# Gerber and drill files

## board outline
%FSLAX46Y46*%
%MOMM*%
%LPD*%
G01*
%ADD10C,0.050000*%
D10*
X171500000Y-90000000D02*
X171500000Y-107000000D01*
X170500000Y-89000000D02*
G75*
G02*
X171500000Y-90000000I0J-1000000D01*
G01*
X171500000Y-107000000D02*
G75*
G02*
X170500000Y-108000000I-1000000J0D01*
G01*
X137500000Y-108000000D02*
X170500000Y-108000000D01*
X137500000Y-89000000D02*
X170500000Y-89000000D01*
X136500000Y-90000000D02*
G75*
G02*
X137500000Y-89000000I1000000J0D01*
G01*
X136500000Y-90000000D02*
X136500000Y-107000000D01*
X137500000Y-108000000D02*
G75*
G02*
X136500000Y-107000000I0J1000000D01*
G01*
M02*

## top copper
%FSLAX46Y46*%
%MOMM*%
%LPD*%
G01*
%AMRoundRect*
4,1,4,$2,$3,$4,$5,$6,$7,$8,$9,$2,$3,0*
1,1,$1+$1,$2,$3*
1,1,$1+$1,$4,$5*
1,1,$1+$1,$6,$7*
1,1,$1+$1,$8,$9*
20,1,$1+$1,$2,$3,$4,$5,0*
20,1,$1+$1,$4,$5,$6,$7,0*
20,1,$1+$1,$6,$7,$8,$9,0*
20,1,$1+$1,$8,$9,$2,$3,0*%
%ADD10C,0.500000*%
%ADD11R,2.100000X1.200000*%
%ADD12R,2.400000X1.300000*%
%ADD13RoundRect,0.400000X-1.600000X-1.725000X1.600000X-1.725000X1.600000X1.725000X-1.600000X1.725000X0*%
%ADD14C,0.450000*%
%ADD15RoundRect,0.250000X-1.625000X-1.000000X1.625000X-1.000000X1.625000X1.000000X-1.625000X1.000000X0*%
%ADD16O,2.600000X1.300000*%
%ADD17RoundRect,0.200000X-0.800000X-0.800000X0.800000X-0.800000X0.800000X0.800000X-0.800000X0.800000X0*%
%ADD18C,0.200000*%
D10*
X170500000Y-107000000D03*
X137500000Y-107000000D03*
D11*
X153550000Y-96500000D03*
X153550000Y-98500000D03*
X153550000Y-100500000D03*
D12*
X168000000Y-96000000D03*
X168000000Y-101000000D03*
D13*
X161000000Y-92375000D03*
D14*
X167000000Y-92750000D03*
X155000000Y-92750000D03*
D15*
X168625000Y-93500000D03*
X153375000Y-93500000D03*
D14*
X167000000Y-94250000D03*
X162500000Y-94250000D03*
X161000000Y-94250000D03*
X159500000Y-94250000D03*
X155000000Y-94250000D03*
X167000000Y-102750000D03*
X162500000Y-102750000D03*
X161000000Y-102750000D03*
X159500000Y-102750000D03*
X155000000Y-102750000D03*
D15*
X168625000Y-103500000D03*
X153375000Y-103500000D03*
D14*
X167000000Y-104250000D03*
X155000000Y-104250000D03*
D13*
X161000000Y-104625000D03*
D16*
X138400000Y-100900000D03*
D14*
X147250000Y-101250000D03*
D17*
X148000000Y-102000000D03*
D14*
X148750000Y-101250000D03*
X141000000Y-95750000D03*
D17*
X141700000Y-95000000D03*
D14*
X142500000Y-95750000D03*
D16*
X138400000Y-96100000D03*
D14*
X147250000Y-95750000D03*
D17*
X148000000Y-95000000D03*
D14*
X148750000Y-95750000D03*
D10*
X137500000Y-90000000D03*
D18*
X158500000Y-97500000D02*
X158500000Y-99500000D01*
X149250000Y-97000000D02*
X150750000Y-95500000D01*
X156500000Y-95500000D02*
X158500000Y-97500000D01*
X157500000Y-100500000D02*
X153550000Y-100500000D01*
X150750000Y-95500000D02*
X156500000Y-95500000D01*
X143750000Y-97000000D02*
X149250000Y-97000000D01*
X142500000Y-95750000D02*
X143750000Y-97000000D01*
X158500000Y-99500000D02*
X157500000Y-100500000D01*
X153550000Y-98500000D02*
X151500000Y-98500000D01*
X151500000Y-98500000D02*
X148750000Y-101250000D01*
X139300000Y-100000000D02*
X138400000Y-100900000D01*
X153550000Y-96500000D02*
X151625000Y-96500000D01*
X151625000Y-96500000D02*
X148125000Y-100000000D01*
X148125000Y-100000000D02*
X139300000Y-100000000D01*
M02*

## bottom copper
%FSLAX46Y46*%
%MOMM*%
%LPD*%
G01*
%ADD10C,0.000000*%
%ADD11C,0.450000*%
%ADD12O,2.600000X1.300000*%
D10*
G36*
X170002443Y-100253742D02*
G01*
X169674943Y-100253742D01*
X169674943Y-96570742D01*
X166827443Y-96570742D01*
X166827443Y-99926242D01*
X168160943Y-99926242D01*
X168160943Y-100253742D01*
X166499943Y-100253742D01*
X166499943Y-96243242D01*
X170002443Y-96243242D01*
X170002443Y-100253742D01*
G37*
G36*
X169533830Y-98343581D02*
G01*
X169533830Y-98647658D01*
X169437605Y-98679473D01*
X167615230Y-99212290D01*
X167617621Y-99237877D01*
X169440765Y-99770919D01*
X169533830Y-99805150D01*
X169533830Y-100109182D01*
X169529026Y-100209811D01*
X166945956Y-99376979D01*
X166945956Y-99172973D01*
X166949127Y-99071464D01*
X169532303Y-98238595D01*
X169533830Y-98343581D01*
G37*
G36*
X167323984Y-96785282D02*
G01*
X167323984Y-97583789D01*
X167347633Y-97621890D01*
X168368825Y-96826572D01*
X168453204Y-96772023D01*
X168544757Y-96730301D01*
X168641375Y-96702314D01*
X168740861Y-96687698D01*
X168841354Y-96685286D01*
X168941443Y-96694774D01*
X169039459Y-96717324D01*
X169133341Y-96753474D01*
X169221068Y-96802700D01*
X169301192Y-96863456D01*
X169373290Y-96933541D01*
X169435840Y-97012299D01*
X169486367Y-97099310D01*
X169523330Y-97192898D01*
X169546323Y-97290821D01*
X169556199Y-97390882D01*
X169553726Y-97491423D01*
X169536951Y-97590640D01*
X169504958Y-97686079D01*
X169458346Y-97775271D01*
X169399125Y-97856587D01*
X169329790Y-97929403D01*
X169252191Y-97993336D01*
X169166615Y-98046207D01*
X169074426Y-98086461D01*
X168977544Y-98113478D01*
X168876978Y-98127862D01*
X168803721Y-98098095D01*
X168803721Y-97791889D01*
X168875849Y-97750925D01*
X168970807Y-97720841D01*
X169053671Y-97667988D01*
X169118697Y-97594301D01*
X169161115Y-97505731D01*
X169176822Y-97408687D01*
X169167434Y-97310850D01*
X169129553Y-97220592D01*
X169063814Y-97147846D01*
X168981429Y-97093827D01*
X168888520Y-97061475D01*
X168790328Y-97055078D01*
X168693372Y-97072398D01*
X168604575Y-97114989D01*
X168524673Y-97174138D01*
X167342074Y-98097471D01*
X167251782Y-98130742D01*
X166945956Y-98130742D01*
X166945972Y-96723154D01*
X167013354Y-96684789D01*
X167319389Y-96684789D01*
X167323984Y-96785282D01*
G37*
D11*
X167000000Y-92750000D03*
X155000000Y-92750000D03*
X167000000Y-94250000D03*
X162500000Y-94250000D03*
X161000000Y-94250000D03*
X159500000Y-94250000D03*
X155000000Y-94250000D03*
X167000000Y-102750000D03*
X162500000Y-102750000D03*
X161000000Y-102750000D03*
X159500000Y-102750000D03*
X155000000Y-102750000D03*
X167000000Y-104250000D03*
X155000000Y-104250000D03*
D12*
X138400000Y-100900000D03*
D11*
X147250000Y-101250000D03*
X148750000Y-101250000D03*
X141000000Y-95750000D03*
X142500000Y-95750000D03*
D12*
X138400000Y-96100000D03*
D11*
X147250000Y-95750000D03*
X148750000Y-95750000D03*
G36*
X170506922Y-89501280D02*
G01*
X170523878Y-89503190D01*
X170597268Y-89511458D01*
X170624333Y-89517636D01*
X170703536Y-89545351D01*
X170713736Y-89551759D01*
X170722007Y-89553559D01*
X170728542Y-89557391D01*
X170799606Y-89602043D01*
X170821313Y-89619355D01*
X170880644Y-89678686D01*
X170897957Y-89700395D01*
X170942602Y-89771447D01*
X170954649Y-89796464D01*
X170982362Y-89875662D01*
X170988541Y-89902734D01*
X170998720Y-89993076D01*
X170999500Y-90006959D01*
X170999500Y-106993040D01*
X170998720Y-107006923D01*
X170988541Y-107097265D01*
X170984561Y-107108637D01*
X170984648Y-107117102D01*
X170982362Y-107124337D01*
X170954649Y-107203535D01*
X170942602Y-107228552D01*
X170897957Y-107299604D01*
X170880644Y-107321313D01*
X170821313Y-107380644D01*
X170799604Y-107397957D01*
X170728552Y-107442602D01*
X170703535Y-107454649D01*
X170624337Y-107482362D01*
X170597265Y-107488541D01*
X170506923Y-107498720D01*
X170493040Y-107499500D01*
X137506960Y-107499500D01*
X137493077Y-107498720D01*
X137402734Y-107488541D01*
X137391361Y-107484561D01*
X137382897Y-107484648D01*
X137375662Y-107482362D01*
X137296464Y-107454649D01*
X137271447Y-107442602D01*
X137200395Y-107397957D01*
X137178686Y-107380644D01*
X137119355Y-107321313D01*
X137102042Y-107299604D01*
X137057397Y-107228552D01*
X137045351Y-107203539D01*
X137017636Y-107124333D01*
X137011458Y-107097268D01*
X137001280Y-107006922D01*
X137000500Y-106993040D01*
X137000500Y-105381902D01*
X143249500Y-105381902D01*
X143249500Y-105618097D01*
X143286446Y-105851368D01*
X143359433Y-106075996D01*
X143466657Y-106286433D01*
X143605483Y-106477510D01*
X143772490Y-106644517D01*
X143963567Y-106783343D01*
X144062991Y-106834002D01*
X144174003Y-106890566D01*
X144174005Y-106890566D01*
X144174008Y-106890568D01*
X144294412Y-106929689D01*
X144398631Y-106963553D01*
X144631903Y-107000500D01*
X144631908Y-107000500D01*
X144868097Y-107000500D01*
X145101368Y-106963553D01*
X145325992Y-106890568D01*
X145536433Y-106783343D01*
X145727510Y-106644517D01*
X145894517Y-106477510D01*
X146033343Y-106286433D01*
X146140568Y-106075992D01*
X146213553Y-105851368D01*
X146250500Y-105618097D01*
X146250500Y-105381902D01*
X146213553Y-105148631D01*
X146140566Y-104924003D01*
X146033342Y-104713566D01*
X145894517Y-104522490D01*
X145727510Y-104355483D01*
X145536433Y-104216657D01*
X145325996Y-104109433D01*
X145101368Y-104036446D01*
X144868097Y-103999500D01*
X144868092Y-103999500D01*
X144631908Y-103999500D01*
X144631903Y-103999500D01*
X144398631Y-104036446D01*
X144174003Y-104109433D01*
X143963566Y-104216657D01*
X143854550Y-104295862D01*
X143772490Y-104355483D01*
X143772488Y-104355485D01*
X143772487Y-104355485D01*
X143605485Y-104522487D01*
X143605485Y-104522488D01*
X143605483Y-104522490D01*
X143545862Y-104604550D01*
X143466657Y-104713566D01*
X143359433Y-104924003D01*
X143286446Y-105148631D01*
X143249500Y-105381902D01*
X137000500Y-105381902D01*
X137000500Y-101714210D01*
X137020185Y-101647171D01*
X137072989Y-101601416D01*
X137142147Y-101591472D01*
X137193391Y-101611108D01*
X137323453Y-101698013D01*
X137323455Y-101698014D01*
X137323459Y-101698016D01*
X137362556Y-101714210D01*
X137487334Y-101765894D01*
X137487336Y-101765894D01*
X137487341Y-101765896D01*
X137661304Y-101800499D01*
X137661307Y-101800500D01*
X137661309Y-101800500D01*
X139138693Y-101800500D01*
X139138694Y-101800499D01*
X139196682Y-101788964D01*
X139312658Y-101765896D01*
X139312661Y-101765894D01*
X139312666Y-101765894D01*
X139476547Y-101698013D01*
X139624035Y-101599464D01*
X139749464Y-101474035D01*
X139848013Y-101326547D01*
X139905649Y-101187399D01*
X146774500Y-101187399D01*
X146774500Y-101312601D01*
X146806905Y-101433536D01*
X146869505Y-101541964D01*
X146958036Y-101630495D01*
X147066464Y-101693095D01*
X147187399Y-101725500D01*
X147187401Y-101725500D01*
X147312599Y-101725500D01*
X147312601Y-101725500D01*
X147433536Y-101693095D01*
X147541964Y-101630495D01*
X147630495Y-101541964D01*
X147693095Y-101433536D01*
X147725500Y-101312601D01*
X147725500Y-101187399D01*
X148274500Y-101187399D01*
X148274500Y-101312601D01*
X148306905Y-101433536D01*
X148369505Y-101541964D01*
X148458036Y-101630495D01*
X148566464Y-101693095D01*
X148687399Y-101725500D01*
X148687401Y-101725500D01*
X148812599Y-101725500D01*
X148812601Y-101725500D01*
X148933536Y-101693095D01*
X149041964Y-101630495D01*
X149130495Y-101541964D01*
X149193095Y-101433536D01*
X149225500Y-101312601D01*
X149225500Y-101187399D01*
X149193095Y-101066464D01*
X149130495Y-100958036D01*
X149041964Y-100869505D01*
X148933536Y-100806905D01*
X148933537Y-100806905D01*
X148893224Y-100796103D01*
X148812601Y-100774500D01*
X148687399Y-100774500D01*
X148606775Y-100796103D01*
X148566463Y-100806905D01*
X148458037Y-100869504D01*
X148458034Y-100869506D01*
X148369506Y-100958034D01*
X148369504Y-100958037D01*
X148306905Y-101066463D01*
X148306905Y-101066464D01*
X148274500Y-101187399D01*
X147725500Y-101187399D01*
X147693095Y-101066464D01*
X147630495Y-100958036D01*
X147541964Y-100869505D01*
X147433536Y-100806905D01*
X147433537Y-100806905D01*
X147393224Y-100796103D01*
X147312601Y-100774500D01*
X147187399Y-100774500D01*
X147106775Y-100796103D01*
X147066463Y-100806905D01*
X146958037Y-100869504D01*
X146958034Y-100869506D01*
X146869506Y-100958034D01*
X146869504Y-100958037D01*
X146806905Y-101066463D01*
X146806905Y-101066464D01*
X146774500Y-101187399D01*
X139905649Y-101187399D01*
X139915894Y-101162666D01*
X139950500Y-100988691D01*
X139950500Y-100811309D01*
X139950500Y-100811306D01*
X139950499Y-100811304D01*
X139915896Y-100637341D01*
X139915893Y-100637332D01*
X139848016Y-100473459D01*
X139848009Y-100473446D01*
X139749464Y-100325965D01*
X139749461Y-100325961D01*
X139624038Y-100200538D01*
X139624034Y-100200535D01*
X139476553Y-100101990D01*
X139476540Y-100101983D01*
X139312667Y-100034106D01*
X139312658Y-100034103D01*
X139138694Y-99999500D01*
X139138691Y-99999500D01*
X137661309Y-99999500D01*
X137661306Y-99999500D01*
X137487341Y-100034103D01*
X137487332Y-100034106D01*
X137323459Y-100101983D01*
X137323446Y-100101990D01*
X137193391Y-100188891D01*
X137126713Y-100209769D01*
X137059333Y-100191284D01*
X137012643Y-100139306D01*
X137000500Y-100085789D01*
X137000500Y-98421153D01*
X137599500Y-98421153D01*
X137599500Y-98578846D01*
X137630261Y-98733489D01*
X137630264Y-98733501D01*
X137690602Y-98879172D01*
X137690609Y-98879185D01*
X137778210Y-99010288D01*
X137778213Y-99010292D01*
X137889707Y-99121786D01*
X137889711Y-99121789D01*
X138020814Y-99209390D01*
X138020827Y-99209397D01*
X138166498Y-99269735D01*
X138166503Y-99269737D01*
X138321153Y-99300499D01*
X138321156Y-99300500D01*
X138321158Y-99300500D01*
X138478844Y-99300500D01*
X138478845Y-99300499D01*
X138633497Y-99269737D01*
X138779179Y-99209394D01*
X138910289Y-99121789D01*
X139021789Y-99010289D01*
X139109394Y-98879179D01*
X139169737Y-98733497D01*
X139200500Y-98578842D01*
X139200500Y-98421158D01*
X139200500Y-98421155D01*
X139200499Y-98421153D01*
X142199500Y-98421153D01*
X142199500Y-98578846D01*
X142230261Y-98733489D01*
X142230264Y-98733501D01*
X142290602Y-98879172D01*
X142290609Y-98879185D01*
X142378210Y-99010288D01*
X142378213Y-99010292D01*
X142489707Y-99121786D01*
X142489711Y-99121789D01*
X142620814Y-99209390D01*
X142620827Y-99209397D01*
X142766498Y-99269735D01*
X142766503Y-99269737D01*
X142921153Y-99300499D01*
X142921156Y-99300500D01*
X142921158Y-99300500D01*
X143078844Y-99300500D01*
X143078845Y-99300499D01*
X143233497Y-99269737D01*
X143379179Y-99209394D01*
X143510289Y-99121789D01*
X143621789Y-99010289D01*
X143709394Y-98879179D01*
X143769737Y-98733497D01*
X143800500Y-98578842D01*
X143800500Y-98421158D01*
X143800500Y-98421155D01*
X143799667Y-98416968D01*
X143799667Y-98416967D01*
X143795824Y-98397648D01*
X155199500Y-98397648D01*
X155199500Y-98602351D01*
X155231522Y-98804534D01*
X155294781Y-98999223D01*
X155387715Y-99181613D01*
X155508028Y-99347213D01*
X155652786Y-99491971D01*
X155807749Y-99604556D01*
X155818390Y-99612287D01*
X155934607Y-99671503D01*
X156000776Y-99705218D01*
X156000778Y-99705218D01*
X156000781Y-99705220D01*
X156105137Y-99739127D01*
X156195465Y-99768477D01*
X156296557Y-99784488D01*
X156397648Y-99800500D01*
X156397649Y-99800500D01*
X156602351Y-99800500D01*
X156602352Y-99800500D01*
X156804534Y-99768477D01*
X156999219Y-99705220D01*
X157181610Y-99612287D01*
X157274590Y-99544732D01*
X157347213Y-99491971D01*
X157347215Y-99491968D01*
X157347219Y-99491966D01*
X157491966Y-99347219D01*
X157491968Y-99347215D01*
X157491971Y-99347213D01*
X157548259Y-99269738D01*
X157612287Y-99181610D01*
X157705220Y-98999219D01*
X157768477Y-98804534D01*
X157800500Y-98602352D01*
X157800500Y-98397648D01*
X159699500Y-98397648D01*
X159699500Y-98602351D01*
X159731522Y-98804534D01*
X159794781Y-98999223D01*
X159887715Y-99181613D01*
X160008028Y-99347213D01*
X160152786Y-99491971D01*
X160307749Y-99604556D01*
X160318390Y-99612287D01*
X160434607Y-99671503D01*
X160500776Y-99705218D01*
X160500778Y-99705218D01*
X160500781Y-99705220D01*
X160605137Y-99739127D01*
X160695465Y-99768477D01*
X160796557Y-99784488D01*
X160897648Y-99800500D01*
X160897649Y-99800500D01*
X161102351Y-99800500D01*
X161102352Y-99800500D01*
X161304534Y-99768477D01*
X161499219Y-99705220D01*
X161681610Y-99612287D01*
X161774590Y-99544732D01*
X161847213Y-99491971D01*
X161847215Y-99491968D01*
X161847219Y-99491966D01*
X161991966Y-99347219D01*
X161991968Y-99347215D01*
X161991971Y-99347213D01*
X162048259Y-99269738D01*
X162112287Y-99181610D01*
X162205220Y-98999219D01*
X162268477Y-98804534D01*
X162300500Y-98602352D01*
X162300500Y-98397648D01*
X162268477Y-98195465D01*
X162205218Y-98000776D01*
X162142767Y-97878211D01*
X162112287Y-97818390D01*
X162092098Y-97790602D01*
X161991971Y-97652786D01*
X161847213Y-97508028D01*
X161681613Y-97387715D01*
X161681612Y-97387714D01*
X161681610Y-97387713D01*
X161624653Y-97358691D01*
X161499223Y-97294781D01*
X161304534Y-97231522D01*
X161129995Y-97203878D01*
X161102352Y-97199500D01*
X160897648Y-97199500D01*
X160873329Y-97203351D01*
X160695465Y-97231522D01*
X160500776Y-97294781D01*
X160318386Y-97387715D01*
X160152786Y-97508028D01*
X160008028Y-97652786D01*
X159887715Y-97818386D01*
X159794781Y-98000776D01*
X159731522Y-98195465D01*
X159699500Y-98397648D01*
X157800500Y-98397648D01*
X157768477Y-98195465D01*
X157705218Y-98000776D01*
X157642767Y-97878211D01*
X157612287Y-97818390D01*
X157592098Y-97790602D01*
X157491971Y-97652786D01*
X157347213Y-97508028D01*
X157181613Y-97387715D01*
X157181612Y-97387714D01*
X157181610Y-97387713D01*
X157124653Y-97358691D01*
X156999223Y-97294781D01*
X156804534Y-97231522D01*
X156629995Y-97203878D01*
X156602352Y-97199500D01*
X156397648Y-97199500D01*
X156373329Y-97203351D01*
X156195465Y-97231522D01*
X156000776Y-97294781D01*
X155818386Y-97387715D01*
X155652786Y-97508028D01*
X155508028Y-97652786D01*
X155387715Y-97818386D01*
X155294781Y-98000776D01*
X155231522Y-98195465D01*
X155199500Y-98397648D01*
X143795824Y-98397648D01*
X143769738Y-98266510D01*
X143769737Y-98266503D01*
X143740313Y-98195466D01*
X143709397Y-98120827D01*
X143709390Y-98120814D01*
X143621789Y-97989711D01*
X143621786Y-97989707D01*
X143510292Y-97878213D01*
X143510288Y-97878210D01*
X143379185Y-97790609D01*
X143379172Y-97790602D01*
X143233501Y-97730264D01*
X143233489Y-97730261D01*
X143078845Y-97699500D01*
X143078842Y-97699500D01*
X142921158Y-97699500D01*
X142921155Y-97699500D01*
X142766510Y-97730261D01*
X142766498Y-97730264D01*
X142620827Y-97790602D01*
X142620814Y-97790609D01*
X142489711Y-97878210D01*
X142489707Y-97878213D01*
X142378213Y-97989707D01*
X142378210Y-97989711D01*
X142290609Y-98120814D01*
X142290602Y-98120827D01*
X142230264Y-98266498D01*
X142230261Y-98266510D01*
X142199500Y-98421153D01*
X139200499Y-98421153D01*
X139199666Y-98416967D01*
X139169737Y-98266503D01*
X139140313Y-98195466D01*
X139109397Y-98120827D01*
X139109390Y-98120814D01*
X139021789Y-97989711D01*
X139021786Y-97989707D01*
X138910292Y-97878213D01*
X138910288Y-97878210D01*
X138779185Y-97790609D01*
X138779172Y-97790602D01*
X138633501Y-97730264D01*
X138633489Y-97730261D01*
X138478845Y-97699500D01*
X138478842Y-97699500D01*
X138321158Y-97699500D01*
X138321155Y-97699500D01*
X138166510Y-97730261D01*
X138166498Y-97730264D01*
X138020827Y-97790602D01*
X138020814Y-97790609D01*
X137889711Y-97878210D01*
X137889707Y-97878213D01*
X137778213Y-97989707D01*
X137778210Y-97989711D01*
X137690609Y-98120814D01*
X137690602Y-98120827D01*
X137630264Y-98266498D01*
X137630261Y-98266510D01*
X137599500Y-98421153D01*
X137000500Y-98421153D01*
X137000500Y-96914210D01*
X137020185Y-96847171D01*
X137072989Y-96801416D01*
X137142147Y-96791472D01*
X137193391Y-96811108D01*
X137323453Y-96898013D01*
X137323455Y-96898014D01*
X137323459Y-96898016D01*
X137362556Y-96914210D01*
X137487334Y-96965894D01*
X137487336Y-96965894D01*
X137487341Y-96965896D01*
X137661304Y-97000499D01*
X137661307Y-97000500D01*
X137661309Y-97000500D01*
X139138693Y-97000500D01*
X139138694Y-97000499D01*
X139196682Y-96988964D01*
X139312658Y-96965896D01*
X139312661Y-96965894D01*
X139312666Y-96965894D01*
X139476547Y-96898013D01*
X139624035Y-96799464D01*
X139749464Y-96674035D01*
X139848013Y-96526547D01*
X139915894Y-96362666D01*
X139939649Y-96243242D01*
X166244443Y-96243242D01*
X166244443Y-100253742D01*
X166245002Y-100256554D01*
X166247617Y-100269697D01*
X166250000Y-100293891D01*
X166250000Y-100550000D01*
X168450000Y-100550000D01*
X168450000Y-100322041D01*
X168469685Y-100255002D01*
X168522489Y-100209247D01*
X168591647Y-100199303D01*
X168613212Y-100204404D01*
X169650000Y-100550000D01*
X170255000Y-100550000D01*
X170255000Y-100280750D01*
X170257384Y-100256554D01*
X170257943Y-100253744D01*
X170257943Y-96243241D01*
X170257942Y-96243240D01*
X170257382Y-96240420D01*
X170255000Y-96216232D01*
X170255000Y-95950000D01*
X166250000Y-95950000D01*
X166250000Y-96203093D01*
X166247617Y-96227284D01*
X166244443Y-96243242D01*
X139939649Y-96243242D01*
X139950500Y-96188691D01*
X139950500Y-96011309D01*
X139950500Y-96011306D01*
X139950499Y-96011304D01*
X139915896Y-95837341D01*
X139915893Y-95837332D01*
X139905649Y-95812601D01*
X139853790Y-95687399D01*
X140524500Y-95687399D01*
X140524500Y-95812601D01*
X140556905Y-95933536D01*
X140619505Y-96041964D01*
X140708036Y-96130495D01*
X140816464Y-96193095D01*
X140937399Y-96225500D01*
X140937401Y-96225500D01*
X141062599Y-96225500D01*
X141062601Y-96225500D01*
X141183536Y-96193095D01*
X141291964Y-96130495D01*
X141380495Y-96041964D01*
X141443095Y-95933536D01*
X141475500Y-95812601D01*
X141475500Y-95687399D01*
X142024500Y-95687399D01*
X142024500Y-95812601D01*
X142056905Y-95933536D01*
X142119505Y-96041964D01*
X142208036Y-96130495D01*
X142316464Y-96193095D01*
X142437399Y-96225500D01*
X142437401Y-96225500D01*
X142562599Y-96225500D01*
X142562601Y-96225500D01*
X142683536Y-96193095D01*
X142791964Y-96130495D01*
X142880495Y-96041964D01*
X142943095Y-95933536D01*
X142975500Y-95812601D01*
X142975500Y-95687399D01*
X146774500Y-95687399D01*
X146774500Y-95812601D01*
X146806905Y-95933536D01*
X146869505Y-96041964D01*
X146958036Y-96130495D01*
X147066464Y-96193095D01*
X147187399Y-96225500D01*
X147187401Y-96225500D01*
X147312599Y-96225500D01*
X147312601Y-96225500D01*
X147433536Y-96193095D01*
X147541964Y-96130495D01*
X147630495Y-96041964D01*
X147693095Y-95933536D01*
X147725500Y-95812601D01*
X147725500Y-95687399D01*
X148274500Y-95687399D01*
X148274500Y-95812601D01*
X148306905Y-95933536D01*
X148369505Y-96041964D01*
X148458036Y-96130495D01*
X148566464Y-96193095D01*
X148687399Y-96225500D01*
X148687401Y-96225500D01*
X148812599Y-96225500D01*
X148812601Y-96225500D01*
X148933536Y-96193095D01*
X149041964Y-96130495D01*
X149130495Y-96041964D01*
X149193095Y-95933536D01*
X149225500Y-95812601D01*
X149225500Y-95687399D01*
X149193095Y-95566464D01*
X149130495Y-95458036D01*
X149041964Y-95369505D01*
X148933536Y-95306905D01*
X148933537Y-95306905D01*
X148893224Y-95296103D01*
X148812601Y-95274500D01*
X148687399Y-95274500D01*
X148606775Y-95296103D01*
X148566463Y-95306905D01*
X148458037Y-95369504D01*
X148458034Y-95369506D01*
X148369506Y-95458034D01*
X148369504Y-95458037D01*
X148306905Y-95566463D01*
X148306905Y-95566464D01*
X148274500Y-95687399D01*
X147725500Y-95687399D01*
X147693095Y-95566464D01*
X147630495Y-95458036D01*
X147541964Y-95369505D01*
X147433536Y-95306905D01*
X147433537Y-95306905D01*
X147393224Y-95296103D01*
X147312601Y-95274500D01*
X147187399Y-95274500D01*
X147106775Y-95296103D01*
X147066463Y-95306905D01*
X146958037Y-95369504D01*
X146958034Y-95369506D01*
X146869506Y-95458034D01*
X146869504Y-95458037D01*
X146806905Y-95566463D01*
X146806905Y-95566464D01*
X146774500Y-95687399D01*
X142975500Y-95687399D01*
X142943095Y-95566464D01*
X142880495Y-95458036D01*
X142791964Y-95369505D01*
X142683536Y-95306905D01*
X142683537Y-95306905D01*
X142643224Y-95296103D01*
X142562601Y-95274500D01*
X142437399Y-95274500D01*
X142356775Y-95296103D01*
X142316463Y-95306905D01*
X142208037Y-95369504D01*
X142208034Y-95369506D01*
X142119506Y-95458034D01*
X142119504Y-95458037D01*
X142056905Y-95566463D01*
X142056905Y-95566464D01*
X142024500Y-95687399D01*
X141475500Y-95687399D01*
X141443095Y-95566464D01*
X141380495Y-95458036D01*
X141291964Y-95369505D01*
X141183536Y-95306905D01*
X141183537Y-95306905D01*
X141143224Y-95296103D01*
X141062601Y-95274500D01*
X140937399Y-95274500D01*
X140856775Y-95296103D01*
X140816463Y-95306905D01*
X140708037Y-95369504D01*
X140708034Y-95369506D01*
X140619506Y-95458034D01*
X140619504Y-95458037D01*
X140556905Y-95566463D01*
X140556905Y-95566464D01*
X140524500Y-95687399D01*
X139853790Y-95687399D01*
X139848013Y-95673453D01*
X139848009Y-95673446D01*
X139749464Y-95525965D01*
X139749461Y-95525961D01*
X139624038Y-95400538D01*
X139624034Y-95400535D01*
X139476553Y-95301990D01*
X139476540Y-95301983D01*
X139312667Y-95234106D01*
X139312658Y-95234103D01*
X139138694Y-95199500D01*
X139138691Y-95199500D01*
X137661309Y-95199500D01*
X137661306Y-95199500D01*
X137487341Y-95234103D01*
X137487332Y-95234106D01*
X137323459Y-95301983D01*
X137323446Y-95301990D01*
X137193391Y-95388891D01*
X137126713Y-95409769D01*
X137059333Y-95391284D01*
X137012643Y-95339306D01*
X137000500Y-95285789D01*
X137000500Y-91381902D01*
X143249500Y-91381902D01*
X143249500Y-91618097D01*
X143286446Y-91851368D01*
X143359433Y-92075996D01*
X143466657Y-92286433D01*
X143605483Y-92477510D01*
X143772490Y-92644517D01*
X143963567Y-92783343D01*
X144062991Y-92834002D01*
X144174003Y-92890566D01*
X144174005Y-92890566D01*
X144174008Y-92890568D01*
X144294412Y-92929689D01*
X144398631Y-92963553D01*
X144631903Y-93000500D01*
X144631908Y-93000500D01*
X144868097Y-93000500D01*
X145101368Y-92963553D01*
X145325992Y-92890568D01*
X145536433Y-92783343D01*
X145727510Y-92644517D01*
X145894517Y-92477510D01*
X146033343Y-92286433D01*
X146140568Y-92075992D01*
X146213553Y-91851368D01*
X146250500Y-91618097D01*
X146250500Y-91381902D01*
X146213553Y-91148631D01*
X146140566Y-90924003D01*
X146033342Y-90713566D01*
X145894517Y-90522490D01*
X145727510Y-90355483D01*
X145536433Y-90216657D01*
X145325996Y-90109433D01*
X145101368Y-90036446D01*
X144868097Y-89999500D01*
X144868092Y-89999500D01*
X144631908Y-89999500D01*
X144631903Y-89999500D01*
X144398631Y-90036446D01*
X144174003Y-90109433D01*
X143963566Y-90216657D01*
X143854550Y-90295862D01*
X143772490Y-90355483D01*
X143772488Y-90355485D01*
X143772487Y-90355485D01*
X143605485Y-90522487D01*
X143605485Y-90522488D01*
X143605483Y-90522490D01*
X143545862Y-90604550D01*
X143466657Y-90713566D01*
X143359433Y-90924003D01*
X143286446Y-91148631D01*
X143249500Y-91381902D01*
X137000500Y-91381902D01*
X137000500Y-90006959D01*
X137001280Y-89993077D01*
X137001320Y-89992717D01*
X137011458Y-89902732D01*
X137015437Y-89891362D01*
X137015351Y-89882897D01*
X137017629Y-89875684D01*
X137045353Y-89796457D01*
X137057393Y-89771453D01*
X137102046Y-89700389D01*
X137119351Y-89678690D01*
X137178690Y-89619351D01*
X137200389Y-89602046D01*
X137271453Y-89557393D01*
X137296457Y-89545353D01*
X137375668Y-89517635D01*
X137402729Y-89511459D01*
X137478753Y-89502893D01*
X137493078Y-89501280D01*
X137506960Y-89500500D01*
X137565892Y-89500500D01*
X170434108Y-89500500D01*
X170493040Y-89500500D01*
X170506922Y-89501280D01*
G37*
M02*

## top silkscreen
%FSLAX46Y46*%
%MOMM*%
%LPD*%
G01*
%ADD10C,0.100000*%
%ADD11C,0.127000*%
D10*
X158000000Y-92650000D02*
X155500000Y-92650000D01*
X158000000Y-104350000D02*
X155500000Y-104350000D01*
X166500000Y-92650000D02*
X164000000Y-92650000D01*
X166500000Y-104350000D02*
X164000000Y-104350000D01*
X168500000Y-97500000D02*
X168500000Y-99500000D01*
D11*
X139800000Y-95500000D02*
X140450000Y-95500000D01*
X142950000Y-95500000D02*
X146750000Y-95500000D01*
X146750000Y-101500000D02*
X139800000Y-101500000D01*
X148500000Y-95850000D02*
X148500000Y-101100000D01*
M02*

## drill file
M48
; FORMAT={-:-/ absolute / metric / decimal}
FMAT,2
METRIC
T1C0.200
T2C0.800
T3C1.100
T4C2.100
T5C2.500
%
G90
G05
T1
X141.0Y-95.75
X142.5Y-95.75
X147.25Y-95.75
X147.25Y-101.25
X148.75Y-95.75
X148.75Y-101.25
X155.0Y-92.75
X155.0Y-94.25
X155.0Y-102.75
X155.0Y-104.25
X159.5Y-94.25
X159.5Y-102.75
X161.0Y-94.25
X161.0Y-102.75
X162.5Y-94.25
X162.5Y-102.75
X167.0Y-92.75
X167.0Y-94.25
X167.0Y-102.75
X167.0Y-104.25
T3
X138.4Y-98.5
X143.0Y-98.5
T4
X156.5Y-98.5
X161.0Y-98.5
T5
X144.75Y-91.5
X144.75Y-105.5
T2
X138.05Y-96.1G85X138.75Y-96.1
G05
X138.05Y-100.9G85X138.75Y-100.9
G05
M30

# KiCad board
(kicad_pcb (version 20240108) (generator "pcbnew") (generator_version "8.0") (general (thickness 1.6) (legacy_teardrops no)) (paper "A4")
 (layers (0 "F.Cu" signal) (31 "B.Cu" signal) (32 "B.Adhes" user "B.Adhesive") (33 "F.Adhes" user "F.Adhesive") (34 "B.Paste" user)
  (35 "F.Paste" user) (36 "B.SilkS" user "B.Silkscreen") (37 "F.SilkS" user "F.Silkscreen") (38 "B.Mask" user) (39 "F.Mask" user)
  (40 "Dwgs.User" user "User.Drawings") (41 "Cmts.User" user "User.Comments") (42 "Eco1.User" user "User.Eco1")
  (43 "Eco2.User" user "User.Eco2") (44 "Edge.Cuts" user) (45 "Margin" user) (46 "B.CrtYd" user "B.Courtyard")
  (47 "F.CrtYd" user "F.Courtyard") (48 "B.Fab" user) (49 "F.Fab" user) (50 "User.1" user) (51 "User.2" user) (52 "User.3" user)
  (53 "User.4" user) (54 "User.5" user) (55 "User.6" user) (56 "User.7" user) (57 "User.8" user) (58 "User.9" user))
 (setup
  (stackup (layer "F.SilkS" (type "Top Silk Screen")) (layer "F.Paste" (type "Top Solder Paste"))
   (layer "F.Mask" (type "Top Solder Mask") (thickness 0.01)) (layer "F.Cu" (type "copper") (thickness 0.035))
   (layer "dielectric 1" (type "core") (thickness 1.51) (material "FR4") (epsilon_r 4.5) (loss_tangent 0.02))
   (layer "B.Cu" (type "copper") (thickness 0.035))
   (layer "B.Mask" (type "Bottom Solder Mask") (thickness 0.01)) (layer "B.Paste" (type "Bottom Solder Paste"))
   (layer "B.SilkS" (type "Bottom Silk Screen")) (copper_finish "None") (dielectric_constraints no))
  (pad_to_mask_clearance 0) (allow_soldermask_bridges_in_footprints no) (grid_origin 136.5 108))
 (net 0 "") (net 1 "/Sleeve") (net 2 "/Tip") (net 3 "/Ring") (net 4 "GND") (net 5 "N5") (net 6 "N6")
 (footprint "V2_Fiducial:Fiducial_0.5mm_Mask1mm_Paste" (layer "F.Cu") (at 170.5 107)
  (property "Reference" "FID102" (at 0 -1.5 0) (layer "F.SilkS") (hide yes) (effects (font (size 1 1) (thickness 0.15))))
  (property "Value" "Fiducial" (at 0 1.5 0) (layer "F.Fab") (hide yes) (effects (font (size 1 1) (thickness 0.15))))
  (pad "" smd circle (at 0 0) (size 0.5 0.5) (layers "F.Cu" "F.Paste" "F.Mask") (solder_mask_margin 0.25) (clearance 0.25)))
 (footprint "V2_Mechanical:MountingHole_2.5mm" (layer "F.Cu") (at 144.75 105.5)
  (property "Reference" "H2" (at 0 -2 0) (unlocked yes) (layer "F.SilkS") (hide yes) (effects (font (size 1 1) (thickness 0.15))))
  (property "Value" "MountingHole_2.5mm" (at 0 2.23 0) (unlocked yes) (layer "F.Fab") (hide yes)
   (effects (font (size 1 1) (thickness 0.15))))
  (pad "" np_thru_hole circle (at 0 0) (size 2.5 2.5) (drill 2.5) (layers "*.Mask")))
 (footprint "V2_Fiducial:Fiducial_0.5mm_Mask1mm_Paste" (layer "F.Cu") (at 137.5 107)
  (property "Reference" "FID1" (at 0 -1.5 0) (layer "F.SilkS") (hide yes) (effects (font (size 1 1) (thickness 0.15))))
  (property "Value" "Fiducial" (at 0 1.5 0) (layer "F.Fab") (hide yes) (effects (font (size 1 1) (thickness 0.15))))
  (pad "" smd circle (at 0 0) (size 0.5 0.5) (layers "F.Cu" "F.Paste" "F.Mask") (solder_mask_margin 0.25) (clearance 0.25)))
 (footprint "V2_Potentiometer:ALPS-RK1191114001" (layer "F.Cu") (at 161 98.5 -90)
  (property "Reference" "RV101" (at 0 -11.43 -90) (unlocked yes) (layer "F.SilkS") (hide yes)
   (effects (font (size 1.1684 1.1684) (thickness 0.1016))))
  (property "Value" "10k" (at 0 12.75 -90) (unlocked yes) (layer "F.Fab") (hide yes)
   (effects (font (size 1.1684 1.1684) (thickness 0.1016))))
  (fp_line (start -5.85 3) (end -5.85 5.5) (stroke (width 0.1) (type solid)) (layer "F.SilkS"))
  (fp_line (start 5.85 3) (end 5.85 5.5) (stroke (width 0.1) (type solid)) (layer "F.SilkS"))
  (fp_line (start -5.85 -5.5) (end -5.85 -3) (stroke (width 0.1) (type solid)) (layer "F.SilkS"))
  (fp_line (start 5.85 -5.5) (end 5.85 -3) (stroke (width 0.1) (type solid)) (layer "F.SilkS"))
  (fp_line (start -1 -7.5) (end 1 -7.5) (stroke (width 0.1) (type solid)) (layer "F.SilkS"))
  (pad "" smd roundrect (at -6.375 0) (size 4 3.75) (layers "F.Paste" "F.Mask") (roundrect_rratio 0.1) (solder_mask_margin 0.1016)
   (zone_connect 2) (thermal_bridge_angle 0))
  (pad "" smd roundrect (at -5 -7.9) (size 3.2 2.5) (layers "F.Paste" "F.Mask") (roundrect_rratio 0.1) (solder_mask_margin 0.1016)
   (zone_connect 2) (thermal_bridge_angle 0))
  (pad "" smd roundrect (at -5 7.9) (size 3.2 2.5) (layers "F.Paste" "F.Mask") (roundrect_rratio 0.1) (solder_mask_margin 0.1016)
   (zone_connect 2) (thermal_bridge_angle 0))
  (pad "" np_thru_hole circle (at 0 0 270) (size 2.1 2.1) (drill 2.1) (layers "*.Cu" "*.Mask"))
  (pad "" np_thru_hole circle (at 0 4.5 270) (size 2.1 2.1) (drill 2.1) (layers "*.Cu" "*.Mask"))
  (pad "" smd roundrect (at 5 -7.9) (size 3.2 2.5) (layers "F.Paste" "F.Mask") (roundrect_rratio 0.1) (solder_mask_margin 0.1016)
   (zone_connect 2) (thermal_bridge_angle 0))
  (pad "" smd roundrect (at 5 7.9) (size 3.2 2.5) (layers "F.Paste" "F.Mask") (roundrect_rratio 0.1) (solder_mask_margin 0.1016)
   (zone_connect 2) (thermal_bridge_angle 0))
  (pad "" smd roundrect (at 6.375 0) (size 4 3.75) (layers "F.Paste" "F.Mask") (roundrect_rratio 0.1) (solder_mask_margin 0.1016)
   (zone_connect 2) (thermal_bridge_angle 0))
  (pad "1" smd rect (at -2 7.45) (size 2.1 1.2) (layers "F.Cu" "F.Paste" "F.Mask") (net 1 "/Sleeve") (solder_mask_margin 0.1016)
   (thermal_bridge_angle 0))
  (pad "2" smd rect (at 0 7.45) (size 2.1 1.2) (layers "F.Cu" "F.Paste" "F.Mask") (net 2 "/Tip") (solder_mask_margin 0.1016)
   (thermal_bridge_angle 0))
  (pad "3" smd rect (at 2 7.45) (size 2.1 1.2) (layers "F.Cu" "F.Paste" "F.Mask") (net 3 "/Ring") (solder_mask_margin 0.1016)
   (thermal_bridge_angle 0))
  (pad "4" smd rect (at -2.5 -7) (size 2.4 1.3) (layers "F.Cu" "F.Paste" "F.Mask") (solder_mask_margin 0.1016) (thermal_bridge_angle 0))
  (pad "5" smd rect (at 2.5 -7) (size 2.4 1.3) (layers "F.Cu" "F.Paste" "F.Mask") (solder_mask_margin 0.1016) (thermal_bridge_angle 0))
  (pad "MP" smd roundrect (at -6.125 0) (size 4 4.25) (layers "F.Cu") (roundrect_rratio 0.1) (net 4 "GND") (solder_mask_margin 0.1016)
   (zone_connect 2) (thermal_bridge_angle 0))
  (pad "MP" thru_hole circle (at -5.75 -6 270) (size 0.45 0.45) (drill 0.2) (layers "*.Cu") (remove_unused_layers yes) (keep_end_layers yes)
   (zone_layer_connections) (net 4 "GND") (solder_mask_margin 0.102))
  (pad "MP" thru_hole circle (at -5.75 6 270) (size 0.45 0.45) (drill 0.2) (layers "*.Cu") (remove_unused_layers yes) (keep_end_layers yes)
   (zone_layer_connections) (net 4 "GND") (solder_mask_margin 0.102))
  (pad "MP" smd roundrect (at -5 -7.625) (size 3.75 2.5) (layers "F.Cu") (roundrect_rratio 0.1) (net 4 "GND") (solder_mask_margin 0.1016)
   (zone_connect 2) (thermal_bridge_angle 0))
  (pad "MP" smd roundrect (at -5 7.625) (size 3.75 2.5) (layers "F.Cu") (roundrect_rratio 0.1) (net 4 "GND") (solder_mask_margin 0.1016)
   (zone_connect 2) (thermal_bridge_angle 0))
  (pad "MP" thru_hole circle (at -4.25 -6 270) (size 0.45 0.45) (drill 0.2) (layers "*.Cu") (remove_unused_layers yes) (keep_end_layers yes)
   (zone_layer_connections) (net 4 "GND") (solder_mask_margin 0.102))
  (pad "MP" thru_hole circle (at -4.25 -1.5 270) (size 0.45 0.45) (drill 0.2) (layers "*.Cu") (remove_unused_layers yes)
   (keep_end_layers yes) (zone_layer_connections) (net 4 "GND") (solder_mask_margin 0.102))
  (pad "MP" thru_hole circle (at -4.25 0 270) (size 0.45 0.45) (drill 0.2) (layers "*.Cu") (remove_unused_layers yes) (keep_end_layers yes)
   (zone_layer_connections) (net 4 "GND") (solder_mask_margin 0.102))
  (pad "MP" thru_hole circle (at -4.25 1.5 270) (size 0.45 0.45) (drill 0.2) (layers "*.Cu") (remove_unused_layers yes)
   (keep_end_layers yes) (zone_layer_connections) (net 4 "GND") (solder_mask_margin 0.102))
  (pad "MP" thru_hole circle (at -4.25 6 270) (size 0.45 0.45) (drill 0.2) (layers "*.Cu") (remove_unused_layers yes) (keep_end_layers yes)
   (zone_layer_connections) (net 4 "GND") (solder_mask_margin 0.102))
  (pad "MP" thru_hole circle (at 4.25 -6 270) (size 0.45 0.45) (drill 0.2) (layers "*.Cu") (remove_unused_layers yes) (keep_end_layers yes)
   (zone_layer_connections) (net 4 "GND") (solder_mask_margin 0.102))
  (pad "MP" thru_hole circle (at 4.25 -1.5 270) (size 0.45 0.45) (drill 0.2) (layers "*.Cu") (remove_unused_layers yes)
   (keep_end_layers yes) (zone_layer_connections) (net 4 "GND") (solder_mask_margin 0.102))
  (pad "MP" thru_hole circle (at 4.25 0 270) (size 0.45 0.45) (drill 0.2) (layers "*.Cu") (remove_unused_layers yes) (keep_end_layers yes)
   (zone_layer_connections) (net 4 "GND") (solder_mask_margin 0.102))
  (pad "MP" thru_hole circle (at 4.25 1.5 270) (size 0.45 0.45) (drill 0.2) (layers "*.Cu") (remove_unused_layers yes) (keep_end_layers yes)
   (zone_layer_connections) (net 4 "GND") (solder_mask_margin 0.102))
  (pad "MP" thru_hole circle (at 4.25 6 270) (size 0.45 0.45) (drill 0.2) (layers "*.Cu") (remove_unused_layers yes) (keep_end_layers yes)
   (zone_layer_connections) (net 4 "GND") (solder_mask_margin 0.102))
  (pad "MP" smd roundrect (at 5 -7.625) (size 3.75 2.5) (layers "F.Cu") (roundrect_rratio 0.1) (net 4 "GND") (solder_mask_margin 0.1016)
   (zone_connect 2) (thermal_bridge_angle 0))
  (pad "MP" smd roundrect (at 5 7.625) (size 3.75 2.5) (layers "F.Cu") (roundrect_rratio 0.1) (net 4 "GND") (solder_mask_margin 0.1016)
   (zone_connect 2) (thermal_bridge_angle 0))
  (pad "MP" thru_hole circle (at 5.75 -6 270) (size 0.45 0.45) (drill 0.2) (layers "*.Cu") (remove_unused_layers yes) (keep_end_layers yes)
   (zone_layer_connections) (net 4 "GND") (solder_mask_margin 0.102))
  (pad "MP" thru_hole circle (at 5.75 6 270) (size 0.45 0.45) (drill 0.2) (layers "*.Cu") (remove_unused_layers yes) (keep_end_layers yes)
   (zone_layer_connections) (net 4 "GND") (solder_mask_margin 0.102))
  (pad "MP" smd roundrect (at 6.125 0) (size 4 4.25) (layers "F.Cu") (roundrect_rratio 0.1) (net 4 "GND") (solder_mask_margin 0.1016)
   (zone_connect 2) (thermal_bridge_angle 0)))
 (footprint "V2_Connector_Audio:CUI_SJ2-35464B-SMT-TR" (layer "F.Cu") (at 142.5 98.5)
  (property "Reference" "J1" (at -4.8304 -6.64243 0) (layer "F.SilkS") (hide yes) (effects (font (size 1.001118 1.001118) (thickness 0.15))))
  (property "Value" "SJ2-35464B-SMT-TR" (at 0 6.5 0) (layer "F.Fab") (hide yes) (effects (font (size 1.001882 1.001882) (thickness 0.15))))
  (fp_line (start -2.7 -3) (end -2.05 -3) (stroke (width 0.127) (type solid)) (layer "F.SilkS"))
  (fp_line (start 0.45 -3) (end 4.25 -3) (stroke (width 0.127) (type solid)) (layer "F.SilkS"))
  (fp_line (start 4.25 3) (end -2.7 3) (stroke (width 0.127) (type solid)) (layer "F.SilkS"))
  (fp_line (start 6 -2.65) (end 6 2.6) (stroke (width 0.127) (type solid)) (layer "F.SilkS"))
  (pad "" np_thru_hole circle (at -4.1 0) (size 1.1 1.1) (drill 1.1) (layers "*.Cu" "*.Mask"))
  (pad "" smd roundrect (at -0.8 -3.7) (size 2 1.6) (layers "F.Mask") (roundrect_rratio 0.1) (solder_mask_margin 0.102))
  (pad "" smd roundrect (at -0.75 -3.825) (size 2.5 1.85) (layers "F.Paste") (roundrect_rratio 0.25) (solder_mask_margin 0.102))
  (pad "" np_thru_hole circle (at 0.5 0) (size 1.1 1.1) (drill 1.1) (layers "*.Cu" "*.Mask"))
  (pad "" smd roundrect (at 5.5 -3.825) (size 2.5 1.85) (layers "F.Paste") (roundrect_rratio 0.25) (solder_mask_margin 0.102))
  (pad "" smd roundrect (at 5.5 -3.7) (size 2 1.6) (layers "F.Mask") (roundrect_rratio 0.1) (solder_mask_margin 0.102))
  (pad "" smd roundrect (at 5.5 3.7) (size 2 1.6) (layers "F.Mask") (roundrect_rratio 0.1) (solder_mask_margin 0.102))
  (pad "" smd roundrect (at 5.5 3.825) (size 2.5 1.85) (layers "F.Paste") (roundrect_rratio 0.25) (solder_mask_margin 0.102))
  (pad "1" thru_hole oval (at -4.1 2.4) (size 2.6 1.3) (drill oval 1.5 0.8) (layers "*.Cu" "F.Paste" "F.Mask") (remove_unused_layers yes)
   (keep_end_layers yes) (zone_layer_connections) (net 1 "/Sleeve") (solder_mask_margin 0.102))
  (pad "2" thru_hole circle (at 4.75 2.75) (size 0.45 0.45) (drill 0.2) (layers "*.Cu") (remove_unused_layers yes) (keep_end_layers yes)
   (zone_layer_connections) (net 2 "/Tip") (solder_mask_margin 0.102))
  (pad "2" smd roundrect (at 5.5 3.5) (size 2 2) (layers "F.Cu") (roundrect_rratio 0.1) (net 2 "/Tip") (solder_mask_margin 0.102))
  (pad "2" thru_hole circle (at 6.25 2.75) (size 0.45 0.45) (drill 0.2) (layers "*.Cu") (remove_unused_layers yes) (keep_end_layers yes)
   (zone_layer_connections) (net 2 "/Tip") (solder_mask_margin 0.102))
  (pad "3" thru_hole circle (at -1.5 -2.75) (size 0.45 0.45) (drill 0.2) (layers "*.Cu") (remove_unused_layers yes) (keep_end_layers yes)
   (zone_layer_connections) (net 3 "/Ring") (solder_mask_margin 0.102))
  (pad "3" smd roundrect (at -0.8 -3.5) (size 2 2) (layers "F.Cu") (roundrect_rratio 0.1) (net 3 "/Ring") (solder_mask_margin 0.102))
  (pad "3" thru_hole circle (at 0 -2.75) (size 0.45 0.45) (drill 0.2) (layers "*.Cu") (remove_unused_layers yes) (keep_end_layers yes)
   (zone_layer_connections) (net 3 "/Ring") (solder_mask_margin 0.102))
  (pad "4" thru_hole oval (at -4.1 -2.4) (size 2.6 1.3) (drill oval 1.5 0.8) (layers "*.Cu" "F.Paste" "F.Mask") (remove_unused_layers yes)
   (keep_end_layers yes) (zone_layer_connections) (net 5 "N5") (solder_mask_margin 0.102))
  (pad "10" thru_hole circle (at 4.75 -2.75) (size 0.45 0.45) (drill 0.2) (layers "*.Cu") (remove_unused_layers yes) (keep_end_layers yes)
   (zone_layer_connections) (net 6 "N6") (solder_mask_margin 0.102))
  (pad "10" smd roundrect (at 5.5 -3.5) (size 2 2) (layers "F.Cu") (roundrect_rratio 0.1) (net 6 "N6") (solder_mask_margin 0.102))
  (pad "10" thru_hole circle (at 6.25 -2.75) (size 0.45 0.45) (drill 0.2) (layers "*.Cu") (remove_unused_layers yes) (keep_end_layers yes)
   (zone_layer_connections) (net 6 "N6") (solder_mask_margin 0.102)))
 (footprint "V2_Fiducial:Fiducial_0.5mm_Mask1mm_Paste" (layer "F.Cu") (at 137.5 90)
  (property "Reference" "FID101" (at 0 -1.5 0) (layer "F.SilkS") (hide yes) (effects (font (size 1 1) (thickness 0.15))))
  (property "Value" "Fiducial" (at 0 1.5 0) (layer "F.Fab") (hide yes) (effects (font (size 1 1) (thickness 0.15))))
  (pad "" smd circle (at 0 0) (size 0.5 0.5) (layers "F.Cu" "F.Paste" "F.Mask") (solder_mask_margin 0.25) (clearance 0.25)))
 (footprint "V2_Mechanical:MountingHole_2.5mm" (layer "F.Cu") (at 144.75 91.5)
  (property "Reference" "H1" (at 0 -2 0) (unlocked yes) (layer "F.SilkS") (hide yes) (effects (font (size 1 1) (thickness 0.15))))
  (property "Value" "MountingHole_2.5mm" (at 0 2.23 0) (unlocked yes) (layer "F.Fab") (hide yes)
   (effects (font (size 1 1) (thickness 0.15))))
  (pad "" np_thru_hole circle (at 0 0) (size 2.5 2.5) (drill 2.5) (layers "*.Mask")))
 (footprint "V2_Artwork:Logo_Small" (layer "B.Cu") (at 168.25 98.25 90)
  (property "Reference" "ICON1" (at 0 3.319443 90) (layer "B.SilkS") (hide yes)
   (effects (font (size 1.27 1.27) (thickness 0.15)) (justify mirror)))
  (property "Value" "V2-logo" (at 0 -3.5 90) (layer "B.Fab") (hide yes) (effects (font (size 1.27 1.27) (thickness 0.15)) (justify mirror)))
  (fp_poly
   (pts (xy 2.006758 -1.750057) (xy -2.003742 -1.750057) (xy -2.003742 -0.089057) (xy -1.676242 -0.089057) (xy -1.676242 -1.422557)
    (xy 1.679258 -1.422557) (xy 1.679258 1.424943) (xy -2.003742 1.424943) (xy -2.003742 1.752443) (xy 2.006758 1.752443))
   (stroke (width 0) (type solid)) (fill solid) (layer "B.Cu"))
  (fp_poly
   (pts (xy -1.520919 1.190765) (xy -0.987877 -0.632379) (xy -0.96229 -0.63477) (xy -0.429473 1.187605) (xy -0.397658 1.28383)
    (xy -0.093581 1.28383) (xy 0.011405 1.282303) (xy -0.821464 -1.300873) (xy -0.922973 -1.304044) (xy -1.126979 -1.304044)
    (xy -1.959811 1.279026) (xy -1.859182 1.28383) (xy -1.55515 1.28383))
   (stroke (width 0) (type solid)) (fill solid) (layer "B.Cu"))
  (fp_poly
   (pts (xy 0.959179 1.296323) (xy 1.057102 1.27333) (xy 1.15069 1.236367) (xy 1.237701 1.18584) (xy 1.316459 1.12329)
    (xy 1.386544 1.051192) (xy 1.4473 0.971068) (xy 1.496526 0.883341) (xy 1.532676 0.789459) (xy 1.555226 0.691443) (xy 1.564714 0.591354)
    (xy 1.562302 0.490861) (xy 1.547686 0.391375) (xy 1.519699 0.294757) (xy 1.477977 0.203204) (xy 1.423428 0.118825)
    (xy 0.62811 -0.902367) (xy 0.666211 -0.926016) (xy 1.464718 -0.926016) (xy 1.565211 -0.930611) (xy 1.565211 -1.236646)
    (xy 1.526846 -1.304028) (xy 0.119258 -1.304044) (xy 0.119258 -0.998218) (xy 0.152529 -0.907926) (xy 1.075862 0.274673)
    (xy 1.135011 0.354575) (xy 1.177602 0.443372) (xy 1.194922 0.540328) (xy 1.188525 0.63852) (xy 1.156173 0.731429) (xy 1.102154 0.813814)
    (xy 1.029408 0.879553) (xy 0.93915 0.917434) (xy 0.841313 0.926822) (xy 0.744269 0.911115) (xy 0.655699 0.868697) (xy 0.582012 0.803671)
    (xy 0.529159 0.720807) (xy 0.499075 0.625849) (xy 0.458111 0.553721) (xy 0.151905 0.553721) (xy 0.122138 0.626978)
    (xy 0.136522 0.727544) (xy 0.163539 0.824426) (xy 0.203793 0.916615) (xy 0.256664 1.002191) (xy 0.320597 1.07979) (xy 0.393413 1.149125)
    (xy 0.474729 1.208346) (xy 0.563921 1.254958) (xy 0.65936 1.286951) (xy 0.758577 1.303726) (xy 0.859118 1.306199))
   (stroke (width 0) (type solid)) (fill solid) (layer "B.Cu"))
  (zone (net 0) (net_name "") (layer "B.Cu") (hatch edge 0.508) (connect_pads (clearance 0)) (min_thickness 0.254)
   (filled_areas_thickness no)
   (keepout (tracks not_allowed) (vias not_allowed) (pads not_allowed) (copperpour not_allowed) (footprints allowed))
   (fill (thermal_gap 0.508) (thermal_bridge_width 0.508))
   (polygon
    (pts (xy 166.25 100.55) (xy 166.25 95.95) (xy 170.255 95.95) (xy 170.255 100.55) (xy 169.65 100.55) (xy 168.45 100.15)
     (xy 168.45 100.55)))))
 (gr_line (start 171.5 90) (end 171.5 107) (stroke (width 0.05) (type solid)) (layer "Edge.Cuts"))
 (gr_arc (start 170.5 89) (mid 171.207107 89.292893) (end 171.5 90) (stroke (width 0.05) (type solid)) (layer "Edge.Cuts"))
 (gr_arc (start 171.5 107) (mid 171.207107 107.707107) (end 170.5 108) (stroke (width 0.05) (type solid)) (layer "Edge.Cuts"))
 (gr_line (start 137.5 108) (end 170.5 108) (stroke (width 0.05) (type solid)) (layer "Edge.Cuts"))
 (gr_line (start 137.5 89) (end 170.5 89) (stroke (width 0.05) (type solid)) (layer "Edge.Cuts"))
 (gr_arc (start 136.5 90) (mid 136.792893 89.292893) (end 137.5 89) (stroke (width 0.05) (type solid)) (layer "Edge.Cuts"))
 (gr_line (start 136.5 90) (end 136.5 107) (stroke (width 0.05) (type solid)) (layer "Edge.Cuts"))
 (gr_arc (start 137.5 108) (mid 136.792893 107.707107) (end 136.5 107) (stroke (width 0.05) (type solid)) (layer "Edge.Cuts"))
 (segment (start 158.5 97.5) (end 158.5 99.5) (width 0.2) (layer "F.Cu") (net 3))
 (segment (start 149.25 97) (end 150.75 95.5) (width 0.2) (layer "F.Cu") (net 3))
 (segment (start 156.5 95.5) (end 158.5 97.5) (width 0.2) (layer "F.Cu") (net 3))
 (segment (start 157.5 100.5) (end 153.55 100.5) (width 0.2) (layer "F.Cu") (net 3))
 (segment (start 150.75 95.5) (end 156.5 95.5) (width 0.2) (layer "F.Cu") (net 3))
 (segment (start 143.75 97) (end 149.25 97) (width 0.2) (layer "F.Cu") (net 3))
 (segment (start 142.5 95.75) (end 143.75 97) (width 0.2) (layer "F.Cu") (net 3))
 (segment (start 158.5 99.5) (end 157.5 100.5) (width 0.2) (layer "F.Cu") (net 3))
 (segment (start 153.55 98.5) (end 151.5 98.5) (width 0.2) (layer "F.Cu") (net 2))
 (segment (start 151.5 98.5) (end 148.75 101.25) (width 0.2) (layer "F.Cu") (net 2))
 (segment (start 139.3 100) (end 138.4 100.9) (width 0.2) (layer "F.Cu") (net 1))
 (segment (start 153.55 96.5) (end 151.625 96.5) (width 0.2) (layer "F.Cu") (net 1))
 (segment (start 151.625 96.5) (end 148.125 100) (width 0.2) (layer "F.Cu") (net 1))
 (segment (start 148.125 100) (end 139.3 100) (width 0.2) (layer "F.Cu") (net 1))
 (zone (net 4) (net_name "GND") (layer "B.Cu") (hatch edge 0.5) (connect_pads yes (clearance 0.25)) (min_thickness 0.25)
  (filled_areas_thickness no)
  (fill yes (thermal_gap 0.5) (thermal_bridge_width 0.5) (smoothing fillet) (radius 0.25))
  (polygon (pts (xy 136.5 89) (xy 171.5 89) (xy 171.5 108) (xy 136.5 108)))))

